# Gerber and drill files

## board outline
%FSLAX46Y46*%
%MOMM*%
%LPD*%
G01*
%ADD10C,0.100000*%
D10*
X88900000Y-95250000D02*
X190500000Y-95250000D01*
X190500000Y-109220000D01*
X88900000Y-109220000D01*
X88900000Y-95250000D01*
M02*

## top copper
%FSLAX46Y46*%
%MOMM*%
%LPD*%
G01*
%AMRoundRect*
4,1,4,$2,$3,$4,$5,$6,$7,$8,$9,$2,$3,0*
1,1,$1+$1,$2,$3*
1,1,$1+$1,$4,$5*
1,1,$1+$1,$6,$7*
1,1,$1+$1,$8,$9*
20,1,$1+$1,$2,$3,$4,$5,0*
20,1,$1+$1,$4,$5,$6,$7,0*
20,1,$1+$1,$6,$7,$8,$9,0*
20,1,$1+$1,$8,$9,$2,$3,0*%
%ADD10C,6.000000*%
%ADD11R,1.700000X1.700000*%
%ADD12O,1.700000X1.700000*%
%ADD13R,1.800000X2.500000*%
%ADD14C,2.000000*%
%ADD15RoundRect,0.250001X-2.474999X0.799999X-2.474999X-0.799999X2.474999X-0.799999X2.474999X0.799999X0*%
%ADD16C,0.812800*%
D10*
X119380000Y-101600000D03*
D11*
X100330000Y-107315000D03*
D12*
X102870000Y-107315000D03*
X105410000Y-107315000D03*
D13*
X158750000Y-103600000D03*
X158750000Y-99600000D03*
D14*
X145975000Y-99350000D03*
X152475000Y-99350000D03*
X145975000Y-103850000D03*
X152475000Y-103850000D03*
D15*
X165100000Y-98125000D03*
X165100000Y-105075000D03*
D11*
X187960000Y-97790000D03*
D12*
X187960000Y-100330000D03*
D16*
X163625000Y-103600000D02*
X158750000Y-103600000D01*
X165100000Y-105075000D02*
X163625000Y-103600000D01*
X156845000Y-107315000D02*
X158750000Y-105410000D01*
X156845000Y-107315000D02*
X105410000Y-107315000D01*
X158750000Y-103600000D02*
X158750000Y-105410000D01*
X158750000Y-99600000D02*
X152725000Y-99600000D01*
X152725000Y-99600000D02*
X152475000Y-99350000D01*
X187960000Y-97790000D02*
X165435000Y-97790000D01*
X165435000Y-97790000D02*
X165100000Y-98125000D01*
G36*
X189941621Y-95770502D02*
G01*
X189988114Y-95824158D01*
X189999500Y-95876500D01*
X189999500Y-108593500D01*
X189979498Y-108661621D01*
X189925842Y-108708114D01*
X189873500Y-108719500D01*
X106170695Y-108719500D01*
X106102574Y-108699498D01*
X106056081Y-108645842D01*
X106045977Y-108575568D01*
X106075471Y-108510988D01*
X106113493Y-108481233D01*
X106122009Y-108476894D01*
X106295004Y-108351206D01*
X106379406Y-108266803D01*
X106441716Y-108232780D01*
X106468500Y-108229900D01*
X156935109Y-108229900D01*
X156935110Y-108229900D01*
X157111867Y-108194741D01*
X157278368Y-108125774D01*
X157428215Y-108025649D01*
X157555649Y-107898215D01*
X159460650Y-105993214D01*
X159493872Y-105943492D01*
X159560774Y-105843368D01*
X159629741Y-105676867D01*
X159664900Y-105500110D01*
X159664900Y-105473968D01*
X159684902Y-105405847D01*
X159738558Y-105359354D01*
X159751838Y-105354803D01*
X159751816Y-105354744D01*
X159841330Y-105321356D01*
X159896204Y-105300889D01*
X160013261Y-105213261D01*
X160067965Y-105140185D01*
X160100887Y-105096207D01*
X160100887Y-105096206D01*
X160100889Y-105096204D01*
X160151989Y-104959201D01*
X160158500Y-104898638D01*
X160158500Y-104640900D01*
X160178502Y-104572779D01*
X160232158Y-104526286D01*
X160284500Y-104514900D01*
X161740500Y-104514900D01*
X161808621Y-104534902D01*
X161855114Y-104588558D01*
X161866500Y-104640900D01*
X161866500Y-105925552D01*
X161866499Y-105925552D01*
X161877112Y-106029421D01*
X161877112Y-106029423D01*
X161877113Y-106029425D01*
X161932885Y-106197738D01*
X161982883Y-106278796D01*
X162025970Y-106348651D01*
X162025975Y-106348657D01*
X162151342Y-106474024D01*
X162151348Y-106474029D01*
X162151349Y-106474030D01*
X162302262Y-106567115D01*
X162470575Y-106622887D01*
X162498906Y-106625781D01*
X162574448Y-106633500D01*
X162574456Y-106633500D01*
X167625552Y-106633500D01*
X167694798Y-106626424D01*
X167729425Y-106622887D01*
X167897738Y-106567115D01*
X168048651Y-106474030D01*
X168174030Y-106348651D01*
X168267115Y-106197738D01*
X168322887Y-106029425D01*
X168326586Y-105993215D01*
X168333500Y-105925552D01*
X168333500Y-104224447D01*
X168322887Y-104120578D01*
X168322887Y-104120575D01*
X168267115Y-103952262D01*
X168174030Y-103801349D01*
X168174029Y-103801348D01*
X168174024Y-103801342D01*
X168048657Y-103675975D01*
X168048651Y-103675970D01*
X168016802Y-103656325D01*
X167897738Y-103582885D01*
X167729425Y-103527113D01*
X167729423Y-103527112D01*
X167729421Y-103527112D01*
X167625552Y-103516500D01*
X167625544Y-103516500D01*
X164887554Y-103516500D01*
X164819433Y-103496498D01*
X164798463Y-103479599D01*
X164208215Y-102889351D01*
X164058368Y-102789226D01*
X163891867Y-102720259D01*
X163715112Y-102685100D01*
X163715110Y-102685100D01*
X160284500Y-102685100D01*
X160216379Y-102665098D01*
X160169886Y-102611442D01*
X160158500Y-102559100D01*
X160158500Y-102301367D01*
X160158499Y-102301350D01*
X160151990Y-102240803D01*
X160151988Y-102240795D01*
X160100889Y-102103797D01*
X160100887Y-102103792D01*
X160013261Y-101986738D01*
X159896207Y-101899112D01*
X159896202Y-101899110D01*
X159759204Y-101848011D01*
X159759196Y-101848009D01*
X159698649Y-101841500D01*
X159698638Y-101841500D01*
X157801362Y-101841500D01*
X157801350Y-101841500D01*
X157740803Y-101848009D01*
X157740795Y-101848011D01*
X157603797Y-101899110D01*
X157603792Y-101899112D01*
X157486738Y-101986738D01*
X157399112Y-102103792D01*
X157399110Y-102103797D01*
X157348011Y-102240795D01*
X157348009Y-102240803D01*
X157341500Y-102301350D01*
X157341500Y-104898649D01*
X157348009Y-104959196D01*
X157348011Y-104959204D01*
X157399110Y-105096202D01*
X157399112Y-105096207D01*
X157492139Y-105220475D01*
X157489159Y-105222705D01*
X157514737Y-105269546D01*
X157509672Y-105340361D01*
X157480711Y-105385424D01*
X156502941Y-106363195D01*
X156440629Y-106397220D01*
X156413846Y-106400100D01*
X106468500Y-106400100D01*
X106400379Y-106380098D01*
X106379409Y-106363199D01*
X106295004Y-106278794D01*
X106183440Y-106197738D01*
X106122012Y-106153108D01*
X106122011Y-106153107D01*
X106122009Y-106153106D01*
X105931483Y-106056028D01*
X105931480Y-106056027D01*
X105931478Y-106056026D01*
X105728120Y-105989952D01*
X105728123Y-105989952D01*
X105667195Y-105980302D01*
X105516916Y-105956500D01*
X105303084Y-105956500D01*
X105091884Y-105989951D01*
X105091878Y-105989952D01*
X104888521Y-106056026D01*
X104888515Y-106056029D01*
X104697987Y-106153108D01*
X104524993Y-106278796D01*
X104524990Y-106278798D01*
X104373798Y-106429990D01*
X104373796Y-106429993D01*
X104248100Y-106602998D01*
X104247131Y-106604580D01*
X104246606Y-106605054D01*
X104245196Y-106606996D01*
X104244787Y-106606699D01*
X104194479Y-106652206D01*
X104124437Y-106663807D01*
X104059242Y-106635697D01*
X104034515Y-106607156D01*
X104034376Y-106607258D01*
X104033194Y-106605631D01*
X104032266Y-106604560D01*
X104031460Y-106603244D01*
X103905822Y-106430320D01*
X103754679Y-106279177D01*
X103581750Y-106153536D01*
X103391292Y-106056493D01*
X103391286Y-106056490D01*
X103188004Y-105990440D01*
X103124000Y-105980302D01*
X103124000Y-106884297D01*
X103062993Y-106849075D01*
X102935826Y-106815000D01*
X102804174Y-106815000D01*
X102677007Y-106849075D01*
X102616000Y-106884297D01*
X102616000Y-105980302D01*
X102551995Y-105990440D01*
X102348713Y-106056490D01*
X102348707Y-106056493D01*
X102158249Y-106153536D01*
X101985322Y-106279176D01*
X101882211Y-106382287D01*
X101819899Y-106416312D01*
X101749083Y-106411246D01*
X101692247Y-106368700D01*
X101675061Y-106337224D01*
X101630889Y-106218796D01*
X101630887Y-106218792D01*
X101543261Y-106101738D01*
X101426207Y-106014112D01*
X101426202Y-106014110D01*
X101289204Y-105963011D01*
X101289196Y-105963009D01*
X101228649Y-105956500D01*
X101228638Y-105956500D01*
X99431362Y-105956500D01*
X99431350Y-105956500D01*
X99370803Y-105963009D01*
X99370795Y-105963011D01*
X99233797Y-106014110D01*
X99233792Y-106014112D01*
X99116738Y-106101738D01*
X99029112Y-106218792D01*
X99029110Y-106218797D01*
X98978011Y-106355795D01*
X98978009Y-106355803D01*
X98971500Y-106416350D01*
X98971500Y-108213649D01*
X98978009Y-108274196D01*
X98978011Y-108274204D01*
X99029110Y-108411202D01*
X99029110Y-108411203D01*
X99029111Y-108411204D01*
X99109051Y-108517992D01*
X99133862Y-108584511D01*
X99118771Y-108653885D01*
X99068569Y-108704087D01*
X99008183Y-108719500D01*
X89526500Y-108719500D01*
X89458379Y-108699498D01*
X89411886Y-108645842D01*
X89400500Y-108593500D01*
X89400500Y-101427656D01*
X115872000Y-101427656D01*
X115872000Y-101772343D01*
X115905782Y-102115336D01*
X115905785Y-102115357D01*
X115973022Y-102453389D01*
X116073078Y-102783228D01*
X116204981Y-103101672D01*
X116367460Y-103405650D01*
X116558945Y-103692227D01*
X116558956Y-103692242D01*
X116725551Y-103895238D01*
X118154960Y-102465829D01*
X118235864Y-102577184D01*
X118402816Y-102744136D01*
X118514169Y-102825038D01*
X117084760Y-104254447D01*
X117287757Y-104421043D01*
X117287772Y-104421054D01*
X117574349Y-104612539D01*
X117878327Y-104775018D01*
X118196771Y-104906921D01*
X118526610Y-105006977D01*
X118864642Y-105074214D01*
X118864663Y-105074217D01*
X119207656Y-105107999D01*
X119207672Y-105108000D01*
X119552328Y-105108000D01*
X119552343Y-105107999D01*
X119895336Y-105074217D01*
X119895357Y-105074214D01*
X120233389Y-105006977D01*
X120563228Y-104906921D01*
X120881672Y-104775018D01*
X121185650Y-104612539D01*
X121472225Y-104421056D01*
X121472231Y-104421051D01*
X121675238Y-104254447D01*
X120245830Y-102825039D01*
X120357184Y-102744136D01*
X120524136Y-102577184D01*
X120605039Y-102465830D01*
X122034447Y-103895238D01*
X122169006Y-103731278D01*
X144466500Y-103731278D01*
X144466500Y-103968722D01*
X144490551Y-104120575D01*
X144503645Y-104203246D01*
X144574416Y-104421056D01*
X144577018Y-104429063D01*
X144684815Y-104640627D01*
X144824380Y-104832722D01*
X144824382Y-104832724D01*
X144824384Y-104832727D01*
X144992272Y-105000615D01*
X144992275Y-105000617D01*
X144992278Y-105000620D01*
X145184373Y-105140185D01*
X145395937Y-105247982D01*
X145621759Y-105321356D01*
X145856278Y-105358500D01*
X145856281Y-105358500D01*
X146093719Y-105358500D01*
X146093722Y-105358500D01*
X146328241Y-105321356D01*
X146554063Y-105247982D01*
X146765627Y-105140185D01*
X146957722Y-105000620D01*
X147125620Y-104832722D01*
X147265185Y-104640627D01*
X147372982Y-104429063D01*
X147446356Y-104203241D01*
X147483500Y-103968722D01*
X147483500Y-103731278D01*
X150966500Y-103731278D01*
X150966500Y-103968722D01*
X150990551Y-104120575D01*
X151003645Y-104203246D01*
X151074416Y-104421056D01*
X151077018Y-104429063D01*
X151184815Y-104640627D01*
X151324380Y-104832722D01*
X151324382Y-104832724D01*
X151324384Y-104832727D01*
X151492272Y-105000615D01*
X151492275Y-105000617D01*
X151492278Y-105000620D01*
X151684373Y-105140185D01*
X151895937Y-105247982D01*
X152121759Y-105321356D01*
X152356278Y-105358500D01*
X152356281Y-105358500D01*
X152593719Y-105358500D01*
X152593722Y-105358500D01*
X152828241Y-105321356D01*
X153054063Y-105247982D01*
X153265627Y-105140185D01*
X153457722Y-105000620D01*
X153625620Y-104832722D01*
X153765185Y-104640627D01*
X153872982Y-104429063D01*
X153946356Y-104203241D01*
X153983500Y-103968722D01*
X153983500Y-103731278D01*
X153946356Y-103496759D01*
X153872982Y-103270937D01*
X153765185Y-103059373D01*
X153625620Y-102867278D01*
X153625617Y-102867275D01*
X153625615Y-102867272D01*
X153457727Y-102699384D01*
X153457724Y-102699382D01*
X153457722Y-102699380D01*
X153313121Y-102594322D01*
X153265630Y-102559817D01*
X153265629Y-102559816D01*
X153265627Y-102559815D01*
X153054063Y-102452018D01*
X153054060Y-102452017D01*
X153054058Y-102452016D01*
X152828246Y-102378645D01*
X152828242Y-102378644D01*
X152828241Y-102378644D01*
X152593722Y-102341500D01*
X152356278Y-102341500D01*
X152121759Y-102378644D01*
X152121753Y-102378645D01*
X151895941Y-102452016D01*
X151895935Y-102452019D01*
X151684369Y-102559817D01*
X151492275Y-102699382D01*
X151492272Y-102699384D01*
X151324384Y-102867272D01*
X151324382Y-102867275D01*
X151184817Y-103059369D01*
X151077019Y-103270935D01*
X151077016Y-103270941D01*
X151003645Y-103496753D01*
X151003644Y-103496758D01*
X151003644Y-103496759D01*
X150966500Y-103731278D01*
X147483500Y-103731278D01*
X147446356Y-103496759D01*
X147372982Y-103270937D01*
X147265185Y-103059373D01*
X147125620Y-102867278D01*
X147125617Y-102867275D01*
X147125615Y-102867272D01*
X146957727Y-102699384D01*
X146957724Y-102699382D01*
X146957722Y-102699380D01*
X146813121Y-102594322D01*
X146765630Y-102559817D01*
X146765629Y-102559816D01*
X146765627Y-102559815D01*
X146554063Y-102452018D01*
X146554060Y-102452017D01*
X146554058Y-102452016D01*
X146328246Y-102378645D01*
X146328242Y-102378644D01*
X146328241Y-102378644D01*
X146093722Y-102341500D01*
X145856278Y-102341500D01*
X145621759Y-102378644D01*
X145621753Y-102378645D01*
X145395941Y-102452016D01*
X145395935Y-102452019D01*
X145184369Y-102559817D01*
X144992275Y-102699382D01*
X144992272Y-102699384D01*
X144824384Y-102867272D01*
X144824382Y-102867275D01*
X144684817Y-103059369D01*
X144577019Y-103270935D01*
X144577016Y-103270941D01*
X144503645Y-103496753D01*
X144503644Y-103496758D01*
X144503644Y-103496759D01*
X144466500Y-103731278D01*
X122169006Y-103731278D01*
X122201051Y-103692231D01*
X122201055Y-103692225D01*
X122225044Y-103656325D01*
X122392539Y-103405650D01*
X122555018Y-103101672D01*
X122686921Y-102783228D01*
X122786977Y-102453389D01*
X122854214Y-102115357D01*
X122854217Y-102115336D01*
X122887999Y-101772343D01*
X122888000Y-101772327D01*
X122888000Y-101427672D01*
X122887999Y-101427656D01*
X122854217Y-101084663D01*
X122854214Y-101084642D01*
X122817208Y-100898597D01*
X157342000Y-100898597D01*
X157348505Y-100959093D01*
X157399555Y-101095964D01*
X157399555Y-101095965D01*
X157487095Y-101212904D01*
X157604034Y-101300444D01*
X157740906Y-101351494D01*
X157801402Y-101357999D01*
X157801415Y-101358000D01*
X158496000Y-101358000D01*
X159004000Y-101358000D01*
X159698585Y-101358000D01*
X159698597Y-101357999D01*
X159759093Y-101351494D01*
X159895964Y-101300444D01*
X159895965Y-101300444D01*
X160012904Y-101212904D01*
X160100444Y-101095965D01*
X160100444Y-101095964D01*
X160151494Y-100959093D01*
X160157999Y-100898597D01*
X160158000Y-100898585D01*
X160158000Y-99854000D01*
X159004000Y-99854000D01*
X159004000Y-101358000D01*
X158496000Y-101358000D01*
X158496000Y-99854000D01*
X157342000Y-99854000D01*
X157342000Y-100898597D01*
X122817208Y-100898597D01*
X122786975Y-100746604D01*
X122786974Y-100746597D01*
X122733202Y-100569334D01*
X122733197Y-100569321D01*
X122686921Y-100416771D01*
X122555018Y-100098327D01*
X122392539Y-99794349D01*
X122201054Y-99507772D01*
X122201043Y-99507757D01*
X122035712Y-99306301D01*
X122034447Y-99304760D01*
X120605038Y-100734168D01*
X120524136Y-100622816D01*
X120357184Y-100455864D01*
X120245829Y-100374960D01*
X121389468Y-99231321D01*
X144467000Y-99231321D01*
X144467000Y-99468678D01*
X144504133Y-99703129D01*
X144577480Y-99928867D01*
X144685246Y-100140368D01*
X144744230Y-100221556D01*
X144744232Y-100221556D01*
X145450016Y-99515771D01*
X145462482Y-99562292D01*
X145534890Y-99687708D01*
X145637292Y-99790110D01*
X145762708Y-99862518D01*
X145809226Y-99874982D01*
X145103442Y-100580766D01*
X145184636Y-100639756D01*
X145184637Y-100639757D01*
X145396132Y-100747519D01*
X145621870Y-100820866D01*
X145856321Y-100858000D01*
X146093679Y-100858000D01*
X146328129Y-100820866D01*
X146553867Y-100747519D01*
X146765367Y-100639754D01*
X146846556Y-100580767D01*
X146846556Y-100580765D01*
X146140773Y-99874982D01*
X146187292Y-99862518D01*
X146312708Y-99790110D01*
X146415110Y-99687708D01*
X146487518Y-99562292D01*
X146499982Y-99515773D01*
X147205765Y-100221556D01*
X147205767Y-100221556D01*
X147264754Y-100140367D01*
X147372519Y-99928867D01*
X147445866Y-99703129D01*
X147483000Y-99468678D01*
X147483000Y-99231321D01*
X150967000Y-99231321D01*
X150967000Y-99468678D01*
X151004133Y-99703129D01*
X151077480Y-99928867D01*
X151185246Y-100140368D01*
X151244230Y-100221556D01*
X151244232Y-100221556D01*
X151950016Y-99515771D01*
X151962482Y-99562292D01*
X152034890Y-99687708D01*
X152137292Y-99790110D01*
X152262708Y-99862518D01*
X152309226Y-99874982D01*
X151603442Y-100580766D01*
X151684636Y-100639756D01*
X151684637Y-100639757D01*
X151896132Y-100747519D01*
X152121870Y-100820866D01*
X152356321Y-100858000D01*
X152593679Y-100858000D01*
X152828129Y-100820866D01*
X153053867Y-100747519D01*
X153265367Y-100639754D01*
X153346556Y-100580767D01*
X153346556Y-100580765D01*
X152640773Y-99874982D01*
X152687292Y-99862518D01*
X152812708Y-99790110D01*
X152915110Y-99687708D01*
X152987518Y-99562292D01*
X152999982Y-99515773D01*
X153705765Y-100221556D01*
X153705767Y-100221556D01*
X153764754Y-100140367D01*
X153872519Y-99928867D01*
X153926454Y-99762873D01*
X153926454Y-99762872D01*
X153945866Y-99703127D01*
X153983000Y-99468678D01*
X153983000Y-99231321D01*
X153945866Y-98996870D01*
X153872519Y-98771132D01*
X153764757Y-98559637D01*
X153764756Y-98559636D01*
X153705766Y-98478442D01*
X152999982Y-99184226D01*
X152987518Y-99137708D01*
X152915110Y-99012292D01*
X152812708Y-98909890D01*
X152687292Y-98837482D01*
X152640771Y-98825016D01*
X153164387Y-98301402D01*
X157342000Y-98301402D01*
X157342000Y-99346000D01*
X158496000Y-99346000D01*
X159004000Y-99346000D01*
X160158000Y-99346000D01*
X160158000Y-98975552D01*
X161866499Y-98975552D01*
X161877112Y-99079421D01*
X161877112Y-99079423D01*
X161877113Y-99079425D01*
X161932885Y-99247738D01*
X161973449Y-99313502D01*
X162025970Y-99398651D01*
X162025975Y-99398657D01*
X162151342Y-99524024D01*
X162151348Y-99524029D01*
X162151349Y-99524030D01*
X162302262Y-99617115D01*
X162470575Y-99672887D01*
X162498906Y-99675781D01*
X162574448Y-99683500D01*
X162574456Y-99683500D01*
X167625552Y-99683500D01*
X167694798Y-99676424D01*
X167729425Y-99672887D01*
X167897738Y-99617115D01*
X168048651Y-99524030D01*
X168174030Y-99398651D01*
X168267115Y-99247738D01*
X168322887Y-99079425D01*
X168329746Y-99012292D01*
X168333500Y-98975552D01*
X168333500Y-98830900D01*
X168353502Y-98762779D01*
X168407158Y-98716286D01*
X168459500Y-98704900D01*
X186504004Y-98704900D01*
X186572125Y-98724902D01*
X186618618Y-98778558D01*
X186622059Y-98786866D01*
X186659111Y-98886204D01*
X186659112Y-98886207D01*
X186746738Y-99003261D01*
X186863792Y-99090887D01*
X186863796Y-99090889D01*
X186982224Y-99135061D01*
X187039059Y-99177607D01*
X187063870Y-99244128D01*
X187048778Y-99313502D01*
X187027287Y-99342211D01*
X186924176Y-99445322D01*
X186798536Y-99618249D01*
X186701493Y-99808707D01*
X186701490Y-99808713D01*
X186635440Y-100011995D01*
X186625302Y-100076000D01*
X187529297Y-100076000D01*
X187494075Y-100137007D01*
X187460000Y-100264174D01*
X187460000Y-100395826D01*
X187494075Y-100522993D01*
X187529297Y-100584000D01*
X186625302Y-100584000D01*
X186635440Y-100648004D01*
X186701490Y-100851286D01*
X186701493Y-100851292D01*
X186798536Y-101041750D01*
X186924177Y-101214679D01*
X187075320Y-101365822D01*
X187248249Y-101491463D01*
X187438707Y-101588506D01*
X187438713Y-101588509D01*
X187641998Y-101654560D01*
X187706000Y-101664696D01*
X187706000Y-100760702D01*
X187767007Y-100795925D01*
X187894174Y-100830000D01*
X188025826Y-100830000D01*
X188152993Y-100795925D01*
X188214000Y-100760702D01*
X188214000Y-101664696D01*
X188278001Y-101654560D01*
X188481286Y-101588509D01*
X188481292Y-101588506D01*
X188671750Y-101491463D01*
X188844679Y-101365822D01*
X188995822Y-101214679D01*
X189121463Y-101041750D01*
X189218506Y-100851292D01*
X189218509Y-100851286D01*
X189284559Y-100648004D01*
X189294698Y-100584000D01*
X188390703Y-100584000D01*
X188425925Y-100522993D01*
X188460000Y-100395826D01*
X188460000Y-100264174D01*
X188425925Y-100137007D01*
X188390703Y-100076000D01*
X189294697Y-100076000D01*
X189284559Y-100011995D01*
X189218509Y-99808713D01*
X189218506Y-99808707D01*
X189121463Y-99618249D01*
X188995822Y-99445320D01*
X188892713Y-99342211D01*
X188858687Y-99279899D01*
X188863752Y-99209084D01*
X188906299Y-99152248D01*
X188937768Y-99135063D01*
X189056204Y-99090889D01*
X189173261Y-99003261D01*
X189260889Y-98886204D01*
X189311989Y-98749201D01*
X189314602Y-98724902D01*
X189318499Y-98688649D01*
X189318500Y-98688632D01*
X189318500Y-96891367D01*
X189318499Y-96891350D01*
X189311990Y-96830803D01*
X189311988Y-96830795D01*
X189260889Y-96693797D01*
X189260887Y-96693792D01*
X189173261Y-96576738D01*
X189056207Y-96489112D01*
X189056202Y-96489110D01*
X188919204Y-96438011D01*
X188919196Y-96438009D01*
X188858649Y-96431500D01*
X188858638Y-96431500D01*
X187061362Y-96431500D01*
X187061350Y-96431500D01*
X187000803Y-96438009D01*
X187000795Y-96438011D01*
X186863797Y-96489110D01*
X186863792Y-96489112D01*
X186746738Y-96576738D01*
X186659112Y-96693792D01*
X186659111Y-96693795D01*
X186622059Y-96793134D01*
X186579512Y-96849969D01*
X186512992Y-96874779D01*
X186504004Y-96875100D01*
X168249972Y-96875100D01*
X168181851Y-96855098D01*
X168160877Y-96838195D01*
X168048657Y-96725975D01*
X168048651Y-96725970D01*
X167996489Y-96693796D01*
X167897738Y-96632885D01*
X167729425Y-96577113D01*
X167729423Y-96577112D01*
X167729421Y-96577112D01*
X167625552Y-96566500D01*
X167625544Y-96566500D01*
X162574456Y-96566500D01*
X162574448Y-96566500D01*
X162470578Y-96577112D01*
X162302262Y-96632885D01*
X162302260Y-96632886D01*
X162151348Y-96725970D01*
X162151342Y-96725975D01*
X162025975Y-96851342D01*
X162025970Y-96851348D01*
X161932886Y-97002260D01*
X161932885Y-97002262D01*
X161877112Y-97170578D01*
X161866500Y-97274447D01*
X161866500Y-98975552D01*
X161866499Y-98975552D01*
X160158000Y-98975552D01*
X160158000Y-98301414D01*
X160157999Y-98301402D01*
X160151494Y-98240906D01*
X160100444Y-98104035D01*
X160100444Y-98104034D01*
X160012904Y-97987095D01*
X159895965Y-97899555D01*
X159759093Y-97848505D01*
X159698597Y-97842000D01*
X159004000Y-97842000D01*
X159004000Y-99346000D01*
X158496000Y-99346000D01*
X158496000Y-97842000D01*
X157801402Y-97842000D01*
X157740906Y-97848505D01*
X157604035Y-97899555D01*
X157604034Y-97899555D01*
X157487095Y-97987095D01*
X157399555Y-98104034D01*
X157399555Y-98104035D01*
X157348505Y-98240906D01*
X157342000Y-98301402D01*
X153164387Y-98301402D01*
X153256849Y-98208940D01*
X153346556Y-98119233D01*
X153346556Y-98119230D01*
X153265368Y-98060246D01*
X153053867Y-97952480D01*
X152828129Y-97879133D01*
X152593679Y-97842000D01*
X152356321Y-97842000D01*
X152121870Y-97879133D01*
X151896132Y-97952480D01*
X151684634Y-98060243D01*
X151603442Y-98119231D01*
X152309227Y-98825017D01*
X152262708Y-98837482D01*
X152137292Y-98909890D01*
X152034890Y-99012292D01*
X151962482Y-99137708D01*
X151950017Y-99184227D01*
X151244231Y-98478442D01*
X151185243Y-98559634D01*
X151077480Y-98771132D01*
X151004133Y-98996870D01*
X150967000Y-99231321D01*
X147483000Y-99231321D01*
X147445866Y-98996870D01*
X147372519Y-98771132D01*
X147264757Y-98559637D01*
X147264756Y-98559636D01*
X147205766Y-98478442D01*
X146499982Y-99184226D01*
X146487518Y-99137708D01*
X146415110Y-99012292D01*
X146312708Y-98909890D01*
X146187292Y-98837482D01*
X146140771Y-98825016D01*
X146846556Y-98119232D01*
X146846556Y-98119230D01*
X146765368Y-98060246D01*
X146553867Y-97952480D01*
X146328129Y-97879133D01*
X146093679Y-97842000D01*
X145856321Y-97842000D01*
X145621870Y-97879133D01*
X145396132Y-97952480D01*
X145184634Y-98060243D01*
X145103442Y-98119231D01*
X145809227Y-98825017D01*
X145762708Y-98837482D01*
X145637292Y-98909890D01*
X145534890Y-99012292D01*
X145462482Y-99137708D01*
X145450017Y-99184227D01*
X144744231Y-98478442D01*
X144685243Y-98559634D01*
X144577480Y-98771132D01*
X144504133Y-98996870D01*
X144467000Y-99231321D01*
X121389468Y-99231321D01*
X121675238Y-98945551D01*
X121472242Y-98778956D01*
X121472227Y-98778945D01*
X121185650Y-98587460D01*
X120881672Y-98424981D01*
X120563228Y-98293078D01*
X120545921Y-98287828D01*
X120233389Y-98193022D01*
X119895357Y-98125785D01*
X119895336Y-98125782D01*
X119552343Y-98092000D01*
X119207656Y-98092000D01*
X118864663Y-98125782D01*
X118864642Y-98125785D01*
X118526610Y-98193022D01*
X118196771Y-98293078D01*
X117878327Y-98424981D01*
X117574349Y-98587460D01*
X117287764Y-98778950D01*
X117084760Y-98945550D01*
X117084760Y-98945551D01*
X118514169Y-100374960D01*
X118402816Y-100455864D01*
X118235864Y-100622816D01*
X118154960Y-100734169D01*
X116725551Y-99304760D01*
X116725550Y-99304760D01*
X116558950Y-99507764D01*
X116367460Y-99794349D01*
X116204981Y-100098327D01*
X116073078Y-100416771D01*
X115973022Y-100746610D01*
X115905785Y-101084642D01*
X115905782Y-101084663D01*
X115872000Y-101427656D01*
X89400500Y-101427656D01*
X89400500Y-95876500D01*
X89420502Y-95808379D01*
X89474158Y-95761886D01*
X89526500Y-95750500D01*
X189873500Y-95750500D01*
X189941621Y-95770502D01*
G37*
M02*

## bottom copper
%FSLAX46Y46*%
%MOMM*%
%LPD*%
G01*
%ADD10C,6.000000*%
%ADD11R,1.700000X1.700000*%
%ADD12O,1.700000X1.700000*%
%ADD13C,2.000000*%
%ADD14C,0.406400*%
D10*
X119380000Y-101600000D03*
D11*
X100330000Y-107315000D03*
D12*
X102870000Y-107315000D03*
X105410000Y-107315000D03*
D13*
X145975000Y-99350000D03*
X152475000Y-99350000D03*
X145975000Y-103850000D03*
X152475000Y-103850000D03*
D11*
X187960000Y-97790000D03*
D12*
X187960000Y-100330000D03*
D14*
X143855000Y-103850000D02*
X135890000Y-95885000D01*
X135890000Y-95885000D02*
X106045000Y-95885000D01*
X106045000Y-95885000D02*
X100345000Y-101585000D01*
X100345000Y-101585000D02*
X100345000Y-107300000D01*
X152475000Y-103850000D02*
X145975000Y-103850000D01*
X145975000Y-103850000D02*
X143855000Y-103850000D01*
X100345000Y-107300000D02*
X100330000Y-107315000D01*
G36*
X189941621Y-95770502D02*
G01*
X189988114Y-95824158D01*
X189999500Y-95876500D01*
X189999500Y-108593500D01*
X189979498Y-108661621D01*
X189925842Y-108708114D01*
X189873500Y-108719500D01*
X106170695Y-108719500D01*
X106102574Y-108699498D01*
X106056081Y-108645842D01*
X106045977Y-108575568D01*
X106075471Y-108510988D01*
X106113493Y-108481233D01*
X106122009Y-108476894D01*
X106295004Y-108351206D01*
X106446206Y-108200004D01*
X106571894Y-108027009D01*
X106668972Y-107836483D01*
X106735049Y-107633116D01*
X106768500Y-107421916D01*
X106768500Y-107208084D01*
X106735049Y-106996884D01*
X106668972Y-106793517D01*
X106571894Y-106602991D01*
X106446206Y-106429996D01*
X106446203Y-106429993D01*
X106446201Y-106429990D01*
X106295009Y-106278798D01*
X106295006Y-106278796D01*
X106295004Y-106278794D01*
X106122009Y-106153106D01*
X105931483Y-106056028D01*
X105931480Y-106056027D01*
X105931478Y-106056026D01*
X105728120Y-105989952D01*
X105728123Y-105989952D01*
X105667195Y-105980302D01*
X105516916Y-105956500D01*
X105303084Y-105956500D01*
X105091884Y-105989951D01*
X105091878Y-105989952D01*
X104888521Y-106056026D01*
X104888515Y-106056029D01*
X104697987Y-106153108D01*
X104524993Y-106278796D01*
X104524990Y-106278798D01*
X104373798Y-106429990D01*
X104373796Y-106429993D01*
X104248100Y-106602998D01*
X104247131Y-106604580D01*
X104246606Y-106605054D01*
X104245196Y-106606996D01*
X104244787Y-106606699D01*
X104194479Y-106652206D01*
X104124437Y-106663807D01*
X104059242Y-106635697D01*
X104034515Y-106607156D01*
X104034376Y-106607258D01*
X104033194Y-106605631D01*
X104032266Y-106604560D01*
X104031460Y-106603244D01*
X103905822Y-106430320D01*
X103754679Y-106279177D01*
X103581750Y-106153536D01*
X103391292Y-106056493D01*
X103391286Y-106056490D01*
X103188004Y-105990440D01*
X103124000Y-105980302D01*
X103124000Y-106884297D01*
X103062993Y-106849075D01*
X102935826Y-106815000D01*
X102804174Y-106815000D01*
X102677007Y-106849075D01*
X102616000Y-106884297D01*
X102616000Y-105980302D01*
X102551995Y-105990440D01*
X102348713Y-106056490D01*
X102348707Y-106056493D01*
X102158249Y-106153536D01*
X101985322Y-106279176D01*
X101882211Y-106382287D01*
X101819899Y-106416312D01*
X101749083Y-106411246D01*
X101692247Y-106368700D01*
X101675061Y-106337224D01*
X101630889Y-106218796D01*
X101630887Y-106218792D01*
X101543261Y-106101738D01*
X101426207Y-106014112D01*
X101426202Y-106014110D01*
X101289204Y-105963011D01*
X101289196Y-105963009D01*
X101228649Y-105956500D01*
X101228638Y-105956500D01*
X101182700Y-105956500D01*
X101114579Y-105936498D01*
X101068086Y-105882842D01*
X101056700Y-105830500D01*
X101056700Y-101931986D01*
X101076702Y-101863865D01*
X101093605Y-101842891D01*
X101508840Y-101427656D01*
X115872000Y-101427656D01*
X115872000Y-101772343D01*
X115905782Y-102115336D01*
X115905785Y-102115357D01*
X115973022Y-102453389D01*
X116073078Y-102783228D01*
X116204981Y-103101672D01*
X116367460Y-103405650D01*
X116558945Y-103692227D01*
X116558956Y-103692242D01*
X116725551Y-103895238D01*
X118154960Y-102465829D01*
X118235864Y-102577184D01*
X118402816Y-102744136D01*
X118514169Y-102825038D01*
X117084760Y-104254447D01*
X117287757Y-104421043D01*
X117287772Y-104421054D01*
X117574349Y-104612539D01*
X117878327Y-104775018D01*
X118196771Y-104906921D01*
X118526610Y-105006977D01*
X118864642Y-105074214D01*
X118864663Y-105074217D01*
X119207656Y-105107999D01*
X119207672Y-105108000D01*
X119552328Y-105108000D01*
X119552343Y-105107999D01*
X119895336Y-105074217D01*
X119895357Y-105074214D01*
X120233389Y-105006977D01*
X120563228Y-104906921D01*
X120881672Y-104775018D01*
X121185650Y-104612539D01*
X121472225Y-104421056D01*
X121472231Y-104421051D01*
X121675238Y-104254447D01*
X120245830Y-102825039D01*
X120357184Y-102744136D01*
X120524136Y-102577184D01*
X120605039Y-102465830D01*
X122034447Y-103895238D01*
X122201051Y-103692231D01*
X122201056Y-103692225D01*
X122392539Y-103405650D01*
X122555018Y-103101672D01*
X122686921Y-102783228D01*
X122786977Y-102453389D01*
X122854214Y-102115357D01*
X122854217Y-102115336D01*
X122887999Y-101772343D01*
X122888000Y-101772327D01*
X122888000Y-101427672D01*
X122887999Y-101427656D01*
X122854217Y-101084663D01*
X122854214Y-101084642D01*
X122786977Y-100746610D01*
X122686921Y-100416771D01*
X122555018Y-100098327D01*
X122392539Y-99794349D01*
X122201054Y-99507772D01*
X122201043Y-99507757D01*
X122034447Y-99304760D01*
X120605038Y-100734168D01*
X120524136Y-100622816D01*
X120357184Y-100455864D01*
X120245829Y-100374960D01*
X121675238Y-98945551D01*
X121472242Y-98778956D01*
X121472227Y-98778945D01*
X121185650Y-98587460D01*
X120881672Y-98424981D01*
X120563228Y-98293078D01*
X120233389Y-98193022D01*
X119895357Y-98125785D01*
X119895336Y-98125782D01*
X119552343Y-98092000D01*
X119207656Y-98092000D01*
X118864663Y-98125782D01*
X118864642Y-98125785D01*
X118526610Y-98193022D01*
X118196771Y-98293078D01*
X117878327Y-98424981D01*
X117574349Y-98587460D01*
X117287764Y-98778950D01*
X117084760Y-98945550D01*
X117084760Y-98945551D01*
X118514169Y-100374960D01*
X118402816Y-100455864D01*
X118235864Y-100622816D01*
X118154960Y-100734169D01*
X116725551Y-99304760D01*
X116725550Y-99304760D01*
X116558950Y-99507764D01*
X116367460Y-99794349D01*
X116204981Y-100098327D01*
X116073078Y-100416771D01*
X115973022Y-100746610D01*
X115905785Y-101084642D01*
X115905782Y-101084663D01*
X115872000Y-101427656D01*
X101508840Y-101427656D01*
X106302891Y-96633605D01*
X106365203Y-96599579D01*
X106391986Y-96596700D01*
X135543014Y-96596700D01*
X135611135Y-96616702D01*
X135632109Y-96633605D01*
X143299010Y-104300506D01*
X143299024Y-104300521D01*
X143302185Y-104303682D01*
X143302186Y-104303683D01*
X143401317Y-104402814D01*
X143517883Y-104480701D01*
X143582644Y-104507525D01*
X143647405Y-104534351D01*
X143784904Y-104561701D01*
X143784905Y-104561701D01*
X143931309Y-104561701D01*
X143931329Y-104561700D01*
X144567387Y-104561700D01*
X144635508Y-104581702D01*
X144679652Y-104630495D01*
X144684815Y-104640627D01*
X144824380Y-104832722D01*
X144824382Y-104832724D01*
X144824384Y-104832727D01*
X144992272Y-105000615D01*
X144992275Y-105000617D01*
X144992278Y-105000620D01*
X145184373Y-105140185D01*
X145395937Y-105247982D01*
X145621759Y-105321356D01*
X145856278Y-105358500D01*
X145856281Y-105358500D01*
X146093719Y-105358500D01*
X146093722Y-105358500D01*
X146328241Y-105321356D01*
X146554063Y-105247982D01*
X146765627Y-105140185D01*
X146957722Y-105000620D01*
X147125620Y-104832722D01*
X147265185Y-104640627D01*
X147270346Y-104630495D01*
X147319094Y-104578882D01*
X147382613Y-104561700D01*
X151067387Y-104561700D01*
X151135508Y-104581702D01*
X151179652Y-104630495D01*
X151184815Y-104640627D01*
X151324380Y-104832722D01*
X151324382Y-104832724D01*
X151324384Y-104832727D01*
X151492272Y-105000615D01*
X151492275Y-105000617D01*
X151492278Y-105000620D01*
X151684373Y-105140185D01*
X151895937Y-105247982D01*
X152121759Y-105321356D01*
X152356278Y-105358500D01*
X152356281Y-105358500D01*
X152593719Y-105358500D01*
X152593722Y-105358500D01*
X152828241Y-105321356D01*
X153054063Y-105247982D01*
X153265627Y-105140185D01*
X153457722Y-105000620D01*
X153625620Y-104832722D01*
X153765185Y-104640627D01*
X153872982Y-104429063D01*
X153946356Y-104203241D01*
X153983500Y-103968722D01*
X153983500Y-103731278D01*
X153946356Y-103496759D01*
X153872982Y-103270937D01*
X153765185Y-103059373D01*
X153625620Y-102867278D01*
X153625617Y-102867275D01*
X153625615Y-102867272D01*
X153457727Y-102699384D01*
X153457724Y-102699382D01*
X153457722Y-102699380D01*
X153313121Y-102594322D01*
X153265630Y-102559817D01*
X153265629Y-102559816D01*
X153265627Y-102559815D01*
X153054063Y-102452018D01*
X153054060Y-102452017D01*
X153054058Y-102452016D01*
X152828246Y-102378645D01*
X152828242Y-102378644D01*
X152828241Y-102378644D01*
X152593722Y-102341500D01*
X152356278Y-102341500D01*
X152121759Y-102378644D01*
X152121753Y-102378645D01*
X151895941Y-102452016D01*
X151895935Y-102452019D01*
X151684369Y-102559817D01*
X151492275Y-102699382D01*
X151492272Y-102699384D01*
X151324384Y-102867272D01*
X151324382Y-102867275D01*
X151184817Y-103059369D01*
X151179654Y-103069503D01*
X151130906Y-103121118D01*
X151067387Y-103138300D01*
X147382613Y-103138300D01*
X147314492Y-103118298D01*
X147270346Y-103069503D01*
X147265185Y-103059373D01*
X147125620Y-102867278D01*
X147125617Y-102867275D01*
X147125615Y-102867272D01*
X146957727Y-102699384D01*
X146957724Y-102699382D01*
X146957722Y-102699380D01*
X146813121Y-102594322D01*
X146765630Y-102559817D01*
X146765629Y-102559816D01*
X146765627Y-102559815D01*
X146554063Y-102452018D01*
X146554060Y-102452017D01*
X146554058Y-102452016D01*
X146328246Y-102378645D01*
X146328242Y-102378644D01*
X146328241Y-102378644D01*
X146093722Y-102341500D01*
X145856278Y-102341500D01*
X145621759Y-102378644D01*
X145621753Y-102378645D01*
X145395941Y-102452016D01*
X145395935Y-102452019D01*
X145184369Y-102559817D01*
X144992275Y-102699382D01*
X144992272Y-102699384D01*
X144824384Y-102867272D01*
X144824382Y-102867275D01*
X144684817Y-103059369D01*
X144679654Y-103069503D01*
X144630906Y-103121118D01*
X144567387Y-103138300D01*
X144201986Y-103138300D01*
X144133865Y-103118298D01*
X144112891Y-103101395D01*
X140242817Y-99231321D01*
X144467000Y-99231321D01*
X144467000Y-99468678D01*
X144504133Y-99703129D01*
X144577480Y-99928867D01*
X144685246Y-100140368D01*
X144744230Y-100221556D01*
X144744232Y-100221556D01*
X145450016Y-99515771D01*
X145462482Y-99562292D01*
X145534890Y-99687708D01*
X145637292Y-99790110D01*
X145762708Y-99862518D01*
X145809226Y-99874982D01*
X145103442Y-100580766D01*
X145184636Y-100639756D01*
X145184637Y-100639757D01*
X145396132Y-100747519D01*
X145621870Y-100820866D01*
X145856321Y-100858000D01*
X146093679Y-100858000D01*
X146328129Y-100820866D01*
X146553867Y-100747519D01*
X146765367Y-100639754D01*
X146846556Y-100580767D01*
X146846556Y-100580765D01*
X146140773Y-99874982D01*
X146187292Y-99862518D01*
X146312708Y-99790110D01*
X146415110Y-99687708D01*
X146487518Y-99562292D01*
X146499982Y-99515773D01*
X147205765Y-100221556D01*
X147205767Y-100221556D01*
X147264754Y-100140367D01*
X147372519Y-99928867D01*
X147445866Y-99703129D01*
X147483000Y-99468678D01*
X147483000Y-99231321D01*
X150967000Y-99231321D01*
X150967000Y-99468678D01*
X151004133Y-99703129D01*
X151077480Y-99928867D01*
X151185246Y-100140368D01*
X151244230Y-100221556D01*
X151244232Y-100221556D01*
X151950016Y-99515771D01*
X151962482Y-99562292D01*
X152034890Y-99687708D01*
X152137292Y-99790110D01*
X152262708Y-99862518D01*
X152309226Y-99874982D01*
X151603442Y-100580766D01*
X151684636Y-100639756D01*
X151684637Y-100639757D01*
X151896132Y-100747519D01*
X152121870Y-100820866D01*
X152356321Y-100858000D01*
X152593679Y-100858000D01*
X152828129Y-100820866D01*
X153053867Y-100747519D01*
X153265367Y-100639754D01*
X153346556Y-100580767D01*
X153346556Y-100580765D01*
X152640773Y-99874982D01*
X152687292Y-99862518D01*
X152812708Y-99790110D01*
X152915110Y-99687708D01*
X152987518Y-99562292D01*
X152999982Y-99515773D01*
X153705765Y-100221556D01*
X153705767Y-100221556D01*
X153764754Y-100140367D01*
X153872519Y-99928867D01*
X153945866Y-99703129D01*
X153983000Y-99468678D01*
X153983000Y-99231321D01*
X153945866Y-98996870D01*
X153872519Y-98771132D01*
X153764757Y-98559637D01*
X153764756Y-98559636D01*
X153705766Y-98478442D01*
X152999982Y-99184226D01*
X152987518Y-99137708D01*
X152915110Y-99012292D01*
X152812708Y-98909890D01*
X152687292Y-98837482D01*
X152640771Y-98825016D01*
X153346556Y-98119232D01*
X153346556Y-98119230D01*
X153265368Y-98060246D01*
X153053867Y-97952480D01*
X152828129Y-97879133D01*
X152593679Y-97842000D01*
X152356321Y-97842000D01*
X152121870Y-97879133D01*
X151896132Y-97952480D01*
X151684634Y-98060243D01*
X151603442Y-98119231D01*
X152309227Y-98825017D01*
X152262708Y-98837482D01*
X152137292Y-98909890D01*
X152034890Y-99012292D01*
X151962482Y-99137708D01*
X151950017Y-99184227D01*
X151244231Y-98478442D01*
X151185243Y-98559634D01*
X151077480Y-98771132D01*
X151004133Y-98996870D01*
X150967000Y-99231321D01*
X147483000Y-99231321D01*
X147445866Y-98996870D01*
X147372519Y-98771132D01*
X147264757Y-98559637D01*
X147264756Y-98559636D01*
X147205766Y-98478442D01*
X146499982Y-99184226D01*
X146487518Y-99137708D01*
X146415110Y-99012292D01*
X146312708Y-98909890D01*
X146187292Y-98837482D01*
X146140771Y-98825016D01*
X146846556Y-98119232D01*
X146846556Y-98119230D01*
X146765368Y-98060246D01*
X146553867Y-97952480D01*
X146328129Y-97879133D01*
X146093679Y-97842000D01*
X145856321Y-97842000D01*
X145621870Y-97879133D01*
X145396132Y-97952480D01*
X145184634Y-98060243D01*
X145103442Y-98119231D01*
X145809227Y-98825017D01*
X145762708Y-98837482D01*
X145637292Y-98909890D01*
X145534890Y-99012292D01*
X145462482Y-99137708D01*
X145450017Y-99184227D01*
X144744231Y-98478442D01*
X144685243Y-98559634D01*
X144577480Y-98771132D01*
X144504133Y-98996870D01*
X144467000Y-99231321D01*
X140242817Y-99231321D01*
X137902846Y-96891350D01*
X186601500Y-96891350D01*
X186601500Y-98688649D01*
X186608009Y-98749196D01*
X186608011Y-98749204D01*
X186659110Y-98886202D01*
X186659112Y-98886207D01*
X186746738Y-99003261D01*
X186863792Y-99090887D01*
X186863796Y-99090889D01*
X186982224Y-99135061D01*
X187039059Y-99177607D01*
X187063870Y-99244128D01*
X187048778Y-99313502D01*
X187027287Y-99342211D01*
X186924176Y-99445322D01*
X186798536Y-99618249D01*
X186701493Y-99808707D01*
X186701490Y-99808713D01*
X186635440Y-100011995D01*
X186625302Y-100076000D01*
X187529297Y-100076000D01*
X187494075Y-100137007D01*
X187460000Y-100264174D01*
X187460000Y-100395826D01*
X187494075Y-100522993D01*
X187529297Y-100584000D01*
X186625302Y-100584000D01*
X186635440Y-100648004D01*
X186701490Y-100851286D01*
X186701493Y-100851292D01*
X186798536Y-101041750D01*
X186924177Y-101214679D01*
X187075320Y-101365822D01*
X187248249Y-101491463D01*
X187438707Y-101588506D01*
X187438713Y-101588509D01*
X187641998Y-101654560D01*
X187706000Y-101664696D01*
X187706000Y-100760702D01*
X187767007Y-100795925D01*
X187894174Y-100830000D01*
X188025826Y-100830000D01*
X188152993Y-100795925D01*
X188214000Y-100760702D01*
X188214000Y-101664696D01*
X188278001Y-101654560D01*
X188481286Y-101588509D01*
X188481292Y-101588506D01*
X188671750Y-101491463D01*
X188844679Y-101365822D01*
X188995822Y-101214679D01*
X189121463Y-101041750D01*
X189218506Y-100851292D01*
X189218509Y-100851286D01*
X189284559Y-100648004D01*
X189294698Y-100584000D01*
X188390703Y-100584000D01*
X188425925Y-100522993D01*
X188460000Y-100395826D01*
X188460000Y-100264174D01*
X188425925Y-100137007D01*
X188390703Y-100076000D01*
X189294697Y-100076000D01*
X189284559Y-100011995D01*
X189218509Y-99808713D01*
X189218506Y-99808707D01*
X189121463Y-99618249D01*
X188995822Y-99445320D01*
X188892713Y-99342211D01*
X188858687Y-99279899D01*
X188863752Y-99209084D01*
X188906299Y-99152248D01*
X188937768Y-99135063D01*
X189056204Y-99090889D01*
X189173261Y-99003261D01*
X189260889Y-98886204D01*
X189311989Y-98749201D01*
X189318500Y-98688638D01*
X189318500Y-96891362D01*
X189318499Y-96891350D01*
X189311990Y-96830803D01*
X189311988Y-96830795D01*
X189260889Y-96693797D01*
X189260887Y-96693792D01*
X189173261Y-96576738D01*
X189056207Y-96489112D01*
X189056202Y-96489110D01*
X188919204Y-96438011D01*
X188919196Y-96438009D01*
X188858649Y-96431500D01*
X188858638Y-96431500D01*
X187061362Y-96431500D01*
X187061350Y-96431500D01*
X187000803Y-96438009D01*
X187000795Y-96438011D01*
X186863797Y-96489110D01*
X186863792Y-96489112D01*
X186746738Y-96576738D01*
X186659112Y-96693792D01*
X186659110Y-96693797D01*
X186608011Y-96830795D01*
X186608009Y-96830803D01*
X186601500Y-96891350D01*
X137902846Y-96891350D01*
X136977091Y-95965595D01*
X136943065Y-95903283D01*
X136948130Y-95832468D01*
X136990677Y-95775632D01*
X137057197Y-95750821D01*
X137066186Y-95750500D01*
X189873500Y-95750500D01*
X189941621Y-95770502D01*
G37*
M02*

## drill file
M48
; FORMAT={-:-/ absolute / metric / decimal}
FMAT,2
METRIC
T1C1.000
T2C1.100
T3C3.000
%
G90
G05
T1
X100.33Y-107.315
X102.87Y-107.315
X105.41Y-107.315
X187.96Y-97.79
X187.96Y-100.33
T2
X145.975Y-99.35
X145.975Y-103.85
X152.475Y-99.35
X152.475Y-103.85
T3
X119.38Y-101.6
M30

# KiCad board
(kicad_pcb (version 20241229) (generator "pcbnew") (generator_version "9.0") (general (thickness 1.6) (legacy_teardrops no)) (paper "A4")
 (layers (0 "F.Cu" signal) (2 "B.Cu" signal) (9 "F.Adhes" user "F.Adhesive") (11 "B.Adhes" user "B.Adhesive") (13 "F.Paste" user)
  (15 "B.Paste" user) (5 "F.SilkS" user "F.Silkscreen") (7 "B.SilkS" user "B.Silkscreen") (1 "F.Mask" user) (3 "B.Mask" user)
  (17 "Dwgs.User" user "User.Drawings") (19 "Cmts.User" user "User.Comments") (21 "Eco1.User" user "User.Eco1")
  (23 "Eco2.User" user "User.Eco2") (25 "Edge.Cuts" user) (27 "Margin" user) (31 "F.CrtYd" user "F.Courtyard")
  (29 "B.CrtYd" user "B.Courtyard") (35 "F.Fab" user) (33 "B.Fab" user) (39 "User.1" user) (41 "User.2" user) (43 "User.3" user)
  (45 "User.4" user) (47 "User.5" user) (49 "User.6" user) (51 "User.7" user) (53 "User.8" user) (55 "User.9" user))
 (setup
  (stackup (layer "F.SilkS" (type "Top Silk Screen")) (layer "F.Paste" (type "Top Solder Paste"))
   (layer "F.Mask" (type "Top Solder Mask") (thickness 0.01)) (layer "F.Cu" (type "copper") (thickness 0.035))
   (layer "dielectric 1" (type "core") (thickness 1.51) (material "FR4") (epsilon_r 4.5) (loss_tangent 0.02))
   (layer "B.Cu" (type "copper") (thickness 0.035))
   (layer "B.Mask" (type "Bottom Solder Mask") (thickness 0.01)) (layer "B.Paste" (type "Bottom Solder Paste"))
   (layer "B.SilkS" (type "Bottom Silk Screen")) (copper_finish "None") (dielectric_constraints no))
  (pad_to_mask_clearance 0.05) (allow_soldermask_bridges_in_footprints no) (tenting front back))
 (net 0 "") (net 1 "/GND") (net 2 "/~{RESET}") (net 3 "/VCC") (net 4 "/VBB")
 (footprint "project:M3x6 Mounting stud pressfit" (layer "F.Cu") (at 119.38 101.6)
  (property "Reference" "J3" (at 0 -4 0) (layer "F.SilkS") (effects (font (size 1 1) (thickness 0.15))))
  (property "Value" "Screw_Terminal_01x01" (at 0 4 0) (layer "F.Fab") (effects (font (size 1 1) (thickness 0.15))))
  (pad "1" thru_hole circle (at 0 0) (size 6 6) (drill 3) (layers "*.Cu" "*.Mask") (remove_unused_layers no) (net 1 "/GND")))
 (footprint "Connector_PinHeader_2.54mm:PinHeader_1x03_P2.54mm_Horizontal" (layer "F.Cu") (at 100.33 107.315 90)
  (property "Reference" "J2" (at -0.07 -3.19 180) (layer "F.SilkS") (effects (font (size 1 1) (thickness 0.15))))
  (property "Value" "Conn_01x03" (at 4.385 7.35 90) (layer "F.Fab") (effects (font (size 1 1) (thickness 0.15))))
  (pad "1" thru_hole rect (at 0 0 90) (size 1.7 1.7) (drill 1) (layers "*.Cu" "*.Mask") (remove_unused_layers no) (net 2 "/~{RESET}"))
  (pad "2" thru_hole oval (at 0 2.54 90) (size 1.7 1.7) (drill 1) (layers "*.Cu" "*.Mask") (remove_unused_layers no) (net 1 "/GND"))
  (pad "3" thru_hole oval (at 0 5.08 90) (size 1.7 1.7) (drill 1) (layers "*.Cu" "*.Mask") (remove_unused_layers no) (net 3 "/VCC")))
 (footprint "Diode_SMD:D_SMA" (layer "F.Cu") (at 158.75 101.6 90)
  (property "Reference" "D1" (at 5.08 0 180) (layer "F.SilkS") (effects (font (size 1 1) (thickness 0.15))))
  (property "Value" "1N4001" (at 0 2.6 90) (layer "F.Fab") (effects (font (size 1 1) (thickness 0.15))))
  (pad "1" smd rect (at -2 0 90) (size 2.5 1.8) (layers "F.Cu" "F.Mask" "F.Paste") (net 3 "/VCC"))
  (pad "2" smd rect (at 2 0 90) (size 2.5 1.8) (layers "F.Cu" "F.Mask" "F.Paste") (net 1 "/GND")))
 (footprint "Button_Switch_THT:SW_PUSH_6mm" (layer "F.Cu") (at 145.975 99.35)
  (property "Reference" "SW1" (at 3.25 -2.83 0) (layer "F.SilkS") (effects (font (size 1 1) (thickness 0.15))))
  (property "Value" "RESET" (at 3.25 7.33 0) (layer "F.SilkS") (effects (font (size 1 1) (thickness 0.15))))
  (pad "1" thru_hole circle (at 0 0 90) (size 2 2) (drill 1.1) (layers "*.Cu" "*.Mask") (remove_unused_layers no) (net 1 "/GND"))
  (pad "1" thru_hole circle (at 6.5 0 90) (size 2 2) (drill 1.1) (layers "*.Cu" "*.Mask") (remove_unused_layers no) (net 1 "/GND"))
  (pad "2" thru_hole circle (at 0 4.5 90) (size 2 2) (drill 1.1) (layers "*.Cu" "*.Mask") (remove_unused_layers no) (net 2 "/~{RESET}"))
  (pad "2" thru_hole circle (at 6.5 4.5 90) (size 2 2) (drill 1.1) (layers "*.Cu" "*.Mask") (remove_unused_layers no) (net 2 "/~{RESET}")))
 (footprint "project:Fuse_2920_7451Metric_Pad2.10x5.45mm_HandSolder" (layer "F.Cu") (at 165.1 101.6 -90)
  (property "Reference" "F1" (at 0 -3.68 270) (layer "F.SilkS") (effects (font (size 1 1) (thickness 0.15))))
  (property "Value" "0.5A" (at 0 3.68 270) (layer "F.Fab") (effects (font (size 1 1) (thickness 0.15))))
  (pad "1" smd roundrect (at -3.475 0 270) (size 2.1 5.45) (layers "F.Cu" "F.Mask" "F.Paste") (roundrect_rratio 0.119048) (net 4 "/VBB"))
  (pad "2" smd roundrect (at 3.475 0 270) (size 2.1 5.45) (layers "F.Cu" "F.Mask" "F.Paste") (roundrect_rratio 0.119048) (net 3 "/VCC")))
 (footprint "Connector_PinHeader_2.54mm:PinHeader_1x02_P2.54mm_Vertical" (layer "B.Cu") (at 187.96 97.79 180)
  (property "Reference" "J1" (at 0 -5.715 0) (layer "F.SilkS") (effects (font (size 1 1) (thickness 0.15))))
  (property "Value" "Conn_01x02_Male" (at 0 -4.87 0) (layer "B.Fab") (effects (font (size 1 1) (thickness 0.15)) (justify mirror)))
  (pad "1" thru_hole rect (at 0 0 180) (size 1.7 1.7) (drill 1) (layers "*.Cu" "*.Mask") (remove_unused_layers no) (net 4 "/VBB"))
  (pad "2" thru_hole oval (at 0 -2.54 180) (size 1.7 1.7) (drill 1) (layers "*.Cu" "*.Mask") (remove_unused_layers no) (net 1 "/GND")))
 (gr_rect (start 88.9 95.25) (end 190.5 109.22) (stroke (width 0.1) (type solid)) (fill no) (layer "Edge.Cuts"))
 (segment (start 163.625 103.6) (end 158.75 103.6) (width 0.8128) (layer "F.Cu") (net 3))
 (segment (start 165.1 105.075) (end 163.625 103.6) (width 0.8128) (layer "F.Cu") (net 3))
 (segment (start 156.845 107.315) (end 158.75 105.41) (width 0.8128) (layer "F.Cu") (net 3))
 (segment (start 156.845 107.315) (end 105.41 107.315) (width 0.8128) (layer "F.Cu") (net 3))
 (segment (start 158.75 103.6) (end 158.75 105.41) (width 0.8128) (layer "F.Cu") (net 3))
 (segment (start 158.75 99.6) (end 152.725 99.6) (width 0.8128) (layer "F.Cu") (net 1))
 (segment (start 152.725 99.6) (end 152.475 99.35) (width 0.8128) (layer "F.Cu") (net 1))
 (segment (start 187.96 97.79) (end 165.435 97.79) (width 0.8128) (layer "F.Cu") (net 4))
 (segment (start 165.435 97.79) (end 165.1 98.125) (width 0.8128) (layer "F.Cu") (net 4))
 (segment (start 143.855 103.85) (end 135.89 95.885) (width 0.4064) (layer "B.Cu") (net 2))
 (segment (start 135.89 95.885) (end 106.045 95.885) (width 0.4064) (layer "B.Cu") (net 2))
 (segment (start 106.045 95.885) (end 100.345 101.585) (width 0.4064) (layer "B.Cu") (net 2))
 (segment (start 100.345 101.585) (end 100.345 107.3) (width 0.4064) (layer "B.Cu") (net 2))
 (segment (start 152.475 103.85) (end 145.975 103.85) (width 0.4064) (layer "B.Cu") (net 2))
 (segment (start 145.975 103.85) (end 143.855 103.85) (width 0.4064) (layer "B.Cu") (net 2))
 (segment (start 100.345 107.3) (end 100.33 107.315) (width 0.4064) (layer "B.Cu") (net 2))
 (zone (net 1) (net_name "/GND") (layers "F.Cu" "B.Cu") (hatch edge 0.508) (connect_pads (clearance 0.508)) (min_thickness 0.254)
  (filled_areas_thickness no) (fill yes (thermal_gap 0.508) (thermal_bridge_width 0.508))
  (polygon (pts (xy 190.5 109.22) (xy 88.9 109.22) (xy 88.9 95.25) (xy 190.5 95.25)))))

